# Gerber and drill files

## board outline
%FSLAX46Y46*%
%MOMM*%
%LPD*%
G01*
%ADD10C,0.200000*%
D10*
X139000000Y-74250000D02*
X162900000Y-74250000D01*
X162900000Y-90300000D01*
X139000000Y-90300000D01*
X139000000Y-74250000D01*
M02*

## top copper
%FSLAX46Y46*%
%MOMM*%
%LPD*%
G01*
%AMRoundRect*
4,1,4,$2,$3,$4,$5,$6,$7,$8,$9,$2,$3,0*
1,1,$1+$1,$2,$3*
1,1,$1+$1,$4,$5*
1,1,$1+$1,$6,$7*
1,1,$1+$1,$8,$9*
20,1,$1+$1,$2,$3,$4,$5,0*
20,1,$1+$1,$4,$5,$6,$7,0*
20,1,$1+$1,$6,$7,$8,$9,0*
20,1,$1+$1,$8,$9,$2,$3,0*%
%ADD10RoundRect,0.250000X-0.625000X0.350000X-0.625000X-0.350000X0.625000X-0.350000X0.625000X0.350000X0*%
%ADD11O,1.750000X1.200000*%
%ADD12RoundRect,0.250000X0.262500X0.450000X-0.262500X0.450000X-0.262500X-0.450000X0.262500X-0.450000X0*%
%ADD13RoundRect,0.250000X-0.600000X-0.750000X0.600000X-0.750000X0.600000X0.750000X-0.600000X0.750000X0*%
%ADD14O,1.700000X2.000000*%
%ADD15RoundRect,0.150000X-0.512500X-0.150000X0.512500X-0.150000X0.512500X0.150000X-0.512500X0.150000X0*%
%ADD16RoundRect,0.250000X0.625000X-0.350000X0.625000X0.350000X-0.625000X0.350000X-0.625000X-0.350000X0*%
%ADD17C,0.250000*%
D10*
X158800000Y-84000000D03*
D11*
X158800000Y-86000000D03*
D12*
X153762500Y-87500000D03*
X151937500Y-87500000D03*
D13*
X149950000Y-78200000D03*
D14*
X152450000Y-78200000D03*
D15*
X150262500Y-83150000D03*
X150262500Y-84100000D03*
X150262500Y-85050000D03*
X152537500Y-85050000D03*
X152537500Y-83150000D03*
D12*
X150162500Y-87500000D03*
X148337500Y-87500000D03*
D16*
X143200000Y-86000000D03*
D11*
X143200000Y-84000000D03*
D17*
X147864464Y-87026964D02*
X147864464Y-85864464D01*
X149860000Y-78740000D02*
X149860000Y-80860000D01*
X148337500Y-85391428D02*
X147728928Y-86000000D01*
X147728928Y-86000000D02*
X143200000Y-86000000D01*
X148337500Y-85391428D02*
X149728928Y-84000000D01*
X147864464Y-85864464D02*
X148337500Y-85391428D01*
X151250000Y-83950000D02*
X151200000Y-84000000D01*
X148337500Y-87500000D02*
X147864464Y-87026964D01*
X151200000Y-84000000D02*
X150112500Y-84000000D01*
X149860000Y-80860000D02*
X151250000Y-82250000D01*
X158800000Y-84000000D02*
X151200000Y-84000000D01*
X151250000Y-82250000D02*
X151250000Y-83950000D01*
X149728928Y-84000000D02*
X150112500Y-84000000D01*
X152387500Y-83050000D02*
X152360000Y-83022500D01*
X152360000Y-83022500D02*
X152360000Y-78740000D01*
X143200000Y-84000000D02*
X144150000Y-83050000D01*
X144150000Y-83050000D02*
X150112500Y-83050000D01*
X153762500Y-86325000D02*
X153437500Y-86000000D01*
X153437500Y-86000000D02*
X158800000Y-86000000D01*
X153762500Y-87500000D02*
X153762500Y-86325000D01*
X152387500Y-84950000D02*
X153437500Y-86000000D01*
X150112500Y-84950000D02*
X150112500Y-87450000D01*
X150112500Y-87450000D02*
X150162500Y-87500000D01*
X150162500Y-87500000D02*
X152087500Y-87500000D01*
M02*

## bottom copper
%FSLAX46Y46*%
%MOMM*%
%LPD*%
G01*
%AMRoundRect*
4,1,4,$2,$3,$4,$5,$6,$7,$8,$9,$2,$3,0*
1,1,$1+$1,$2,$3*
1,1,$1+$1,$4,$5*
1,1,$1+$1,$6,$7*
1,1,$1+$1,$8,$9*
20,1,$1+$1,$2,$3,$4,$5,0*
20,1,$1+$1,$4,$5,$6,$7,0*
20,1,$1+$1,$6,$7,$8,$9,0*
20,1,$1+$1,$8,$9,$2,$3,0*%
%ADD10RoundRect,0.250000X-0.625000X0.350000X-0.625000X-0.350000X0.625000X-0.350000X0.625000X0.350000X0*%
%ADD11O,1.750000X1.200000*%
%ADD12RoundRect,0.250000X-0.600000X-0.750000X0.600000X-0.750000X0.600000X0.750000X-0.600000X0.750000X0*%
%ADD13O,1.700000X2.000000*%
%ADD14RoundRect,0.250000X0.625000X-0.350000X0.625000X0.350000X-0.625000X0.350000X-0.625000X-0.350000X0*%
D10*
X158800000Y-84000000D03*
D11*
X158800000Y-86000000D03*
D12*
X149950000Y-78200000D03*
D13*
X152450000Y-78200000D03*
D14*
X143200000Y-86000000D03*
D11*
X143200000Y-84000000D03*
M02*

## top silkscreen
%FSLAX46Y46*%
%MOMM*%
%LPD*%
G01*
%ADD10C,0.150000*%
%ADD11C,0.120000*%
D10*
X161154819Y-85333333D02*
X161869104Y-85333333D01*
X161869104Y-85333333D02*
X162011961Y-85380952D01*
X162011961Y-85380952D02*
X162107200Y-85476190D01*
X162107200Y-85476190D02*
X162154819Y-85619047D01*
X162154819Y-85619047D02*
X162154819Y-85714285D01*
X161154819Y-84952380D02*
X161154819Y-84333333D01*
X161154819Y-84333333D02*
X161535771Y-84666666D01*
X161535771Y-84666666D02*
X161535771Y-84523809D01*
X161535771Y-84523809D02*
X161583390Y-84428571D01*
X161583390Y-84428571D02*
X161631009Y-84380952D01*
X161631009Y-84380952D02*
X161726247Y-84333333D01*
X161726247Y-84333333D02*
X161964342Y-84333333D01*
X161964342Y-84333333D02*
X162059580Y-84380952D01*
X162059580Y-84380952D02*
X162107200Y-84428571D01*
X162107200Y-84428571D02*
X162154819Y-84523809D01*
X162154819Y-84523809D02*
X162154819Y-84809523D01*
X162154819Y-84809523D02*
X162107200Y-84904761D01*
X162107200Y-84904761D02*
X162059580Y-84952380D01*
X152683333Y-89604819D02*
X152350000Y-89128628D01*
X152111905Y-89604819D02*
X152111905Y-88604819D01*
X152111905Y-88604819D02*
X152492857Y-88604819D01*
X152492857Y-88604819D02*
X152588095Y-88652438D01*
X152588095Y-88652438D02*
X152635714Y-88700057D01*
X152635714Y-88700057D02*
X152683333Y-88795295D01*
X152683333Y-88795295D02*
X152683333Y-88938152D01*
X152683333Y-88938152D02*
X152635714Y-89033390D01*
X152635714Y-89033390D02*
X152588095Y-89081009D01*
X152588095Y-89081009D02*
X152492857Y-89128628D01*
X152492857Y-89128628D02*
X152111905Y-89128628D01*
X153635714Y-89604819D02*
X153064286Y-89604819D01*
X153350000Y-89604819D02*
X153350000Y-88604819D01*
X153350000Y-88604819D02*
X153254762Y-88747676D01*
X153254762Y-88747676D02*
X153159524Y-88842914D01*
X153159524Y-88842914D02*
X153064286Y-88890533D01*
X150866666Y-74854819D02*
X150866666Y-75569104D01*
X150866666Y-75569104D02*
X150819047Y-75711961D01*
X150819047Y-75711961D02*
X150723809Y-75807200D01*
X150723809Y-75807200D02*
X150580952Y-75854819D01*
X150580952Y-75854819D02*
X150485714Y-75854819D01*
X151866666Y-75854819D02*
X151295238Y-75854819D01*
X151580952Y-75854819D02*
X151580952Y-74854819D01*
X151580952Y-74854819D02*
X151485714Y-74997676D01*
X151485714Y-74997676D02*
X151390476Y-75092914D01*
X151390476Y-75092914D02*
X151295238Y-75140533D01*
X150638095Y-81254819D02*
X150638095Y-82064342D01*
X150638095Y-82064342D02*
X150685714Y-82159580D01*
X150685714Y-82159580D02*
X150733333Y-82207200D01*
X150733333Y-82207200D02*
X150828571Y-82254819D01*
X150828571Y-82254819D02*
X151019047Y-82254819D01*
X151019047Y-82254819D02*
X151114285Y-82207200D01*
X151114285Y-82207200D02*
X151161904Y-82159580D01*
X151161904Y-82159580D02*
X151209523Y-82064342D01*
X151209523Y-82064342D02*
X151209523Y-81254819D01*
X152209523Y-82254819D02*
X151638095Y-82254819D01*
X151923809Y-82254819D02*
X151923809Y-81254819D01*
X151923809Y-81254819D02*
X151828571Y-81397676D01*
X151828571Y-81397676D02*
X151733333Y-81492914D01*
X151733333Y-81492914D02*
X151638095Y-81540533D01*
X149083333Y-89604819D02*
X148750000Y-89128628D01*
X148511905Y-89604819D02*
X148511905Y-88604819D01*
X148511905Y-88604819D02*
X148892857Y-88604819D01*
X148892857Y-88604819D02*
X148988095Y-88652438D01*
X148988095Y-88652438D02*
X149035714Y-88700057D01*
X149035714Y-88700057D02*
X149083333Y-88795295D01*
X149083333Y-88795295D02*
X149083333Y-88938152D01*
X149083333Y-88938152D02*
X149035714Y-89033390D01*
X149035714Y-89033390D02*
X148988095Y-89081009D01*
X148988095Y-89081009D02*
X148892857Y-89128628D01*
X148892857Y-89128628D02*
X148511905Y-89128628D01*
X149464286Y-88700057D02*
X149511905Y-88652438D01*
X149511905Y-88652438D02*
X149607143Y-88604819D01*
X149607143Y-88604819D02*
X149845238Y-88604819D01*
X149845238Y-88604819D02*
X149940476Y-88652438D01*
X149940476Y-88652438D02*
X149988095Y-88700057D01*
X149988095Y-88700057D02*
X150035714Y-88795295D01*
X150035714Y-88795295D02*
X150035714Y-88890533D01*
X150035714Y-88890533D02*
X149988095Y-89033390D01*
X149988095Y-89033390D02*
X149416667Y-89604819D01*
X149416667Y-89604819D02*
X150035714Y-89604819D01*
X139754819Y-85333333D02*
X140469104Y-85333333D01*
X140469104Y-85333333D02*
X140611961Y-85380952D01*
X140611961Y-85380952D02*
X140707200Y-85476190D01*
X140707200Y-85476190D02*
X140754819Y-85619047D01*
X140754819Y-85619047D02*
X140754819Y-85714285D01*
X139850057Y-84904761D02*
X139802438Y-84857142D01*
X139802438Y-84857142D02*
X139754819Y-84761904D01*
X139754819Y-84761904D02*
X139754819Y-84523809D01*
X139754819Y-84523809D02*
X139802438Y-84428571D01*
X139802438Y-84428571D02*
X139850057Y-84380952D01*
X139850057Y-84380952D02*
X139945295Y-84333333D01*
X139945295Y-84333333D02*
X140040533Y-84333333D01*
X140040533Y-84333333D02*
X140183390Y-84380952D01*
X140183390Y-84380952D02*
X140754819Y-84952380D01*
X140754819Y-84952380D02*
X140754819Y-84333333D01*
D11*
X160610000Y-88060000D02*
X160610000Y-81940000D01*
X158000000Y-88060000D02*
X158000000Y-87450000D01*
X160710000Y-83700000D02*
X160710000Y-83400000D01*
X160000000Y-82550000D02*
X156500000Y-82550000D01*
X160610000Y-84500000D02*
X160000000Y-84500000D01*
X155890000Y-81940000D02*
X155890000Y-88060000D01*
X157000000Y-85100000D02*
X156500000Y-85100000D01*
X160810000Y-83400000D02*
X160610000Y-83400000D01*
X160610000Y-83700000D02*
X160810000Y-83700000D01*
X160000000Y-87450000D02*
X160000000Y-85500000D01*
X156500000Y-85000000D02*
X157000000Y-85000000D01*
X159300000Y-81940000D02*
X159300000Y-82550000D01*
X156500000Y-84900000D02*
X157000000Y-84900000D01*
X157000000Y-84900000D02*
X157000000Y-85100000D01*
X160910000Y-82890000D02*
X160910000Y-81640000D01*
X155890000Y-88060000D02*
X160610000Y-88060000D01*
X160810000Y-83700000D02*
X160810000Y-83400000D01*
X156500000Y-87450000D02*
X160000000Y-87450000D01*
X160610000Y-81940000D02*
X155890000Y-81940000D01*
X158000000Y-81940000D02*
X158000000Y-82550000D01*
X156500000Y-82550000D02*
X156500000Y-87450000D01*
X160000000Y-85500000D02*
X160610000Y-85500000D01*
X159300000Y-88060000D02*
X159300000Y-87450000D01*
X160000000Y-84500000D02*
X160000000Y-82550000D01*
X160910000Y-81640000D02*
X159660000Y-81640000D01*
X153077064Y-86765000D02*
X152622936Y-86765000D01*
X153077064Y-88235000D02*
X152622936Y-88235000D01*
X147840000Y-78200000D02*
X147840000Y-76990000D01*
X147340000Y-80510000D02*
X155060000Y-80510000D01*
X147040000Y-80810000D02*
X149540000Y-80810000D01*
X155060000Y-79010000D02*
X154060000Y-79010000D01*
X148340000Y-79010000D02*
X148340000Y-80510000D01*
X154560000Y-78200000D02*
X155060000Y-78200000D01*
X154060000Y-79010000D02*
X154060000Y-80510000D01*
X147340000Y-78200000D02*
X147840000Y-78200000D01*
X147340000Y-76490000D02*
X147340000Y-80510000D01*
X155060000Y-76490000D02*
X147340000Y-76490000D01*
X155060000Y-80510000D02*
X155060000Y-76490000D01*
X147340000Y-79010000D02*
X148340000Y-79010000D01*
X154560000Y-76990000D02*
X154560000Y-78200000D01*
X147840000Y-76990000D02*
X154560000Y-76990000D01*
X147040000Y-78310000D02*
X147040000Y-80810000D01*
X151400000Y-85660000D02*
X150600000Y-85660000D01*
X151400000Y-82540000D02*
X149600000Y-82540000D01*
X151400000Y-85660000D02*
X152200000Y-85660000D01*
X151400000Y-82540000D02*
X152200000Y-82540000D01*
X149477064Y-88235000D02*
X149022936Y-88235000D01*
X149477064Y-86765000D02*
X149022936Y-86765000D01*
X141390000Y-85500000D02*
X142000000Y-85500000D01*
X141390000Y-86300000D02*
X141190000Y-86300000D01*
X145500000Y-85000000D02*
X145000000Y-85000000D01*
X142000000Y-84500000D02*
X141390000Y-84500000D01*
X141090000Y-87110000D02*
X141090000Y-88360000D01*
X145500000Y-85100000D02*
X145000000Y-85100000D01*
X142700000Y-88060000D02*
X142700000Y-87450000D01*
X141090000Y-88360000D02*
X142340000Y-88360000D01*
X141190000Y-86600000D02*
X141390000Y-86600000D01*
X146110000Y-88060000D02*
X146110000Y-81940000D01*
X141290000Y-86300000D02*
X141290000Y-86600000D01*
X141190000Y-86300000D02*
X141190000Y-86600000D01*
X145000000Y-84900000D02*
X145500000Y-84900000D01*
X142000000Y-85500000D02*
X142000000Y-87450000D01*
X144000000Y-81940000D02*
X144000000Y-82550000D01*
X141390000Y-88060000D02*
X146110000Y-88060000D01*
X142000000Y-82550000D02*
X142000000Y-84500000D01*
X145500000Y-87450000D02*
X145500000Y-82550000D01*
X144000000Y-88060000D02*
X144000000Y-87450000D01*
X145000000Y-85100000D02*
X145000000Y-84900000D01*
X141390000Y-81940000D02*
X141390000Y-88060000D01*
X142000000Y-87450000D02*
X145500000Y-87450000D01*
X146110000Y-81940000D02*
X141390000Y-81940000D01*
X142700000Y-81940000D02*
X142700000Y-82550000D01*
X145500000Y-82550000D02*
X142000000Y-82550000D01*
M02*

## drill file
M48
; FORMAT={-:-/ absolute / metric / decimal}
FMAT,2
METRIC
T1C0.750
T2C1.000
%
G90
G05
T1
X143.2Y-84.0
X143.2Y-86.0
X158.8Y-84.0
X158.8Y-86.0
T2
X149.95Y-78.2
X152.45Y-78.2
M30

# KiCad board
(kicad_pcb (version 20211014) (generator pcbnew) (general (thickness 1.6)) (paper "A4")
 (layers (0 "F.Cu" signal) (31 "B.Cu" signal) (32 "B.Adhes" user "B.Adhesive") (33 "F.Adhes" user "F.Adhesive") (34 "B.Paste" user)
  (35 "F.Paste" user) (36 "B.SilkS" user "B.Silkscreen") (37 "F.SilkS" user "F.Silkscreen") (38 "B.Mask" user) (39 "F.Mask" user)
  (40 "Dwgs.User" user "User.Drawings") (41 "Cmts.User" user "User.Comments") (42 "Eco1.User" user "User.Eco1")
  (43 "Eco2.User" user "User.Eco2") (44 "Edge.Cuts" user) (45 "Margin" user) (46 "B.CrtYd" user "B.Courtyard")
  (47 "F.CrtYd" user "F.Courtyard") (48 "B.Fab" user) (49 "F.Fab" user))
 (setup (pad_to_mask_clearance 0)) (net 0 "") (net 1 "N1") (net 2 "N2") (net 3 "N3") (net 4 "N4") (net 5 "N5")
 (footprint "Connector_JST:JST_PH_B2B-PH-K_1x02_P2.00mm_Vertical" (layer "F.Cu") (at 158.8 84 -90)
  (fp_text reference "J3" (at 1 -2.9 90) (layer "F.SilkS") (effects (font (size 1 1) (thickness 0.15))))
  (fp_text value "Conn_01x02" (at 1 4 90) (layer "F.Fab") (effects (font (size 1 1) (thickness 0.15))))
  (fp_line (start 4.06 -1.81) (end -2.06 -1.81) (layer "F.SilkS") (width 0.12))
  (fp_line (start 4.06 0.8) (end 3.45 0.8) (layer "F.SilkS") (width 0.12))
  (fp_line (start -0.3 -1.91) (end -0.6 -1.91) (layer "F.SilkS") (width 0.12))
  (fp_line (start -1.45 -1.2) (end -1.45 2.3) (layer "F.SilkS") (width 0.12))
  (fp_line (start 0.5 -1.81) (end 0.5 -1.2) (layer "F.SilkS") (width 0.12))
  (fp_line (start -2.06 2.91) (end 4.06 2.91) (layer "F.SilkS") (width 0.12))
  (fp_line (start 1.1 1.8) (end 1.1 2.3) (layer "F.SilkS") (width 0.12))
  (fp_line (start -0.6 -2.01) (end -0.6 -1.81) (layer "F.SilkS") (width 0.12))
  (fp_line (start -0.3 -1.81) (end -0.3 -2.01) (layer "F.SilkS") (width 0.12))
  (fp_line (start 3.45 -1.2) (end 1.5 -1.2) (layer "F.SilkS") (width 0.12))
  (fp_line (start 1 2.3) (end 1 1.8) (layer "F.SilkS") (width 0.12))
  (fp_line (start -2.06 -0.5) (end -1.45 -0.5) (layer "F.SilkS") (width 0.12))
  (fp_line (start 0.9 2.3) (end 0.9 1.8) (layer "F.SilkS") (width 0.12))
  (fp_line (start 0.9 1.8) (end 1.1 1.8) (layer "F.SilkS") (width 0.12))
  (fp_line (start -1.11 -2.11) (end -2.36 -2.11) (layer "F.SilkS") (width 0.12))
  (fp_line (start 4.06 2.91) (end 4.06 -1.81) (layer "F.SilkS") (width 0.12))
  (fp_line (start -0.3 -2.01) (end -0.6 -2.01) (layer "F.SilkS") (width 0.12))
  (fp_line (start 3.45 2.3) (end 3.45 -1.2) (layer "F.SilkS") (width 0.12))
  (fp_line (start -2.06 -1.81) (end -2.06 2.91) (layer "F.SilkS") (width 0.12))
  (fp_line (start -2.06 0.8) (end -1.45 0.8) (layer "F.SilkS") (width 0.12))
  (fp_line (start -1.45 2.3) (end 3.45 2.3) (layer "F.SilkS") (width 0.12))
  (fp_line (start 1.5 -1.2) (end 1.5 -1.81) (layer "F.SilkS") (width 0.12))
  (fp_line (start 4.06 -0.5) (end 3.45 -0.5) (layer "F.SilkS") (width 0.12))
  (fp_line (start 0.5 -1.2) (end -1.45 -1.2) (layer "F.SilkS") (width 0.12))
  (fp_line (start -2.36 -2.11) (end -2.36 -0.86) (layer "F.SilkS") (width 0.12))
  (pad "1" thru_hole roundrect locked (at 0 0 270) (size 1.2 1.75) (drill 0.75) (layers *.Cu *.Mask) (roundrect_rratio 0.208333)
   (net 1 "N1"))
  (pad "2" thru_hole oval locked (at 2 0 270) (size 1.2 1.75) (drill 0.75) (layers *.Cu *.Mask) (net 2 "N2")))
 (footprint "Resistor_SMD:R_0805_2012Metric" (layer "F.Cu") (at 152.85 87.5 180)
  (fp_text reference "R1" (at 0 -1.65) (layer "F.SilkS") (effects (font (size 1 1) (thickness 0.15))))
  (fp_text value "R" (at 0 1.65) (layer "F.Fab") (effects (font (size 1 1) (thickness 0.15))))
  (fp_line (start -0.227064 0.735) (end 0.227064 0.735) (layer "F.SilkS") (width 0.12))
  (fp_line (start -0.227064 -0.735) (end 0.227064 -0.735) (layer "F.SilkS") (width 0.12))
  (pad "1" smd roundrect locked (at -0.9125 0 180) (size 1.025 1.4) (layers "F.Cu" "F.Paste" "F.Mask") (roundrect_rratio 0.243902)
   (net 2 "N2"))
  (pad "2" smd roundrect locked (at 0.9125 0 180) (size 1.025 1.4) (layers "F.Cu" "F.Paste" "F.Mask") (roundrect_rratio 0.243902)
   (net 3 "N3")))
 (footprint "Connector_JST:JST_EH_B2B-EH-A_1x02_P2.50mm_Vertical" (layer "F.Cu") (at 149.95 78.2)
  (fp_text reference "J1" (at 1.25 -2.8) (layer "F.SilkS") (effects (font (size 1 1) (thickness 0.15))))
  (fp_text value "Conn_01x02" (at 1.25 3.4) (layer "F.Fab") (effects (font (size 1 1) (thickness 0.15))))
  (fp_line (start -2.11 0) (end -2.11 -1.21) (layer "F.SilkS") (width 0.12))
  (fp_line (start -2.61 2.31) (end 5.11 2.31) (layer "F.SilkS") (width 0.12))
  (fp_line (start -2.91 2.61) (end -0.41 2.61) (layer "F.SilkS") (width 0.12))
  (fp_line (start 5.11 0.81) (end 4.11 0.81) (layer "F.SilkS") (width 0.12))
  (fp_line (start -1.61 0.81) (end -1.61 2.31) (layer "F.SilkS") (width 0.12))
  (fp_line (start 4.61 0) (end 5.11 0) (layer "F.SilkS") (width 0.12))
  (fp_line (start 4.11 0.81) (end 4.11 2.31) (layer "F.SilkS") (width 0.12))
  (fp_line (start -2.61 0) (end -2.11 0) (layer "F.SilkS") (width 0.12))
  (fp_line (start -2.61 -1.71) (end -2.61 2.31) (layer "F.SilkS") (width 0.12))
  (fp_line (start 5.11 -1.71) (end -2.61 -1.71) (layer "F.SilkS") (width 0.12))
  (fp_line (start 5.11 2.31) (end 5.11 -1.71) (layer "F.SilkS") (width 0.12))
  (fp_line (start -2.61 0.81) (end -1.61 0.81) (layer "F.SilkS") (width 0.12))
  (fp_line (start 4.61 -1.21) (end 4.61 0) (layer "F.SilkS") (width 0.12))
  (fp_line (start -2.11 -1.21) (end 4.61 -1.21) (layer "F.SilkS") (width 0.12))
  (fp_line (start -2.91 0.11) (end -2.91 2.61) (layer "F.SilkS") (width 0.12))
  (pad "1" thru_hole roundrect locked (at 0 0) (size 1.7 2) (drill 1) (layers *.Cu *.Mask) (roundrect_rratio 0.147059) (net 1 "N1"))
  (pad "2" thru_hole oval locked (at 2.5 0) (size 1.7 2) (drill 1) (layers *.Cu *.Mask) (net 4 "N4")))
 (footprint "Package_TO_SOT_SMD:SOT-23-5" (layer "F.Cu") (at 151.4 84.1)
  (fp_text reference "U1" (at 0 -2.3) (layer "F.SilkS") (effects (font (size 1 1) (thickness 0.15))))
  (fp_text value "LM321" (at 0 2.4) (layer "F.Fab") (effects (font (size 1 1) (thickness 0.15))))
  (fp_line (start 0 1.56) (end -0.8 1.56) (layer "F.SilkS") (width 0.12))
  (fp_line (start 0 -1.56) (end -1.8 -1.56) (layer "F.SilkS") (width 0.12))
  (fp_line (start 0 1.56) (end 0.8 1.56) (layer "F.SilkS") (width 0.12))
  (fp_line (start 0 -1.56) (end 0.8 -1.56) (layer "F.SilkS") (width 0.12))
  (pad "1" smd roundrect locked (at -1.1375 -0.95) (size 1.325 0.6) (layers "F.Cu" "F.Paste" "F.Mask") (roundrect_rratio 0.25) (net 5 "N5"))
  (pad "2" smd roundrect locked (at -1.1375 0) (size 1.325 0.6) (layers "F.Cu" "F.Paste" "F.Mask") (roundrect_rratio 0.25) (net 1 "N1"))
  (pad "3" smd roundrect locked (at -1.1375 0.95) (size 1.325 0.6) (layers "F.Cu" "F.Paste" "F.Mask") (roundrect_rratio 0.25) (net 3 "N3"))
  (pad "4" smd roundrect locked (at 1.1375 0.95) (size 1.325 0.6) (layers "F.Cu" "F.Paste" "F.Mask") (roundrect_rratio 0.25) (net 2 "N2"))
  (pad "5" smd roundrect locked (at 1.1375 -0.95) (size 1.325 0.6) (layers "F.Cu" "F.Paste" "F.Mask") (roundrect_rratio 0.25) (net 4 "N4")))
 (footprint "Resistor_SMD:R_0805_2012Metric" (layer "F.Cu") (at 149.25 87.5 180)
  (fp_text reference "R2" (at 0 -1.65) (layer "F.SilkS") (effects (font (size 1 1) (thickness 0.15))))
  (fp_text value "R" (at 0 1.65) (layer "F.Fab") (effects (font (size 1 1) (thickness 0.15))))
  (fp_line (start -0.227064 -0.735) (end 0.227064 -0.735) (layer "F.SilkS") (width 0.12))
  (fp_line (start -0.227064 0.735) (end 0.227064 0.735) (layer "F.SilkS") (width 0.12))
  (pad "1" smd roundrect locked (at -0.9125 0 180) (size 1.025 1.4) (layers "F.Cu" "F.Paste" "F.Mask") (roundrect_rratio 0.243902)
   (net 3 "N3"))
  (pad "2" smd roundrect locked (at 0.9125 0 180) (size 1.025 1.4) (layers "F.Cu" "F.Paste" "F.Mask") (roundrect_rratio 0.243902)
   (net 1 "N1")))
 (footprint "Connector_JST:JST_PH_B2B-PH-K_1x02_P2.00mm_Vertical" (layer "F.Cu") (at 143.2 86 90)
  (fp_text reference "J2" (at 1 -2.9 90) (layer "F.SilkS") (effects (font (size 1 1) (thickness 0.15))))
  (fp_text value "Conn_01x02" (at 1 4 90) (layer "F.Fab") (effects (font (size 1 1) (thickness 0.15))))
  (fp_line (start 0.5 -1.81) (end 0.5 -1.2) (layer "F.SilkS") (width 0.12))
  (fp_line (start -0.3 -1.81) (end -0.3 -2.01) (layer "F.SilkS") (width 0.12))
  (fp_line (start 1 2.3) (end 1 1.8) (layer "F.SilkS") (width 0.12))
  (fp_line (start 1.5 -1.2) (end 1.5 -1.81) (layer "F.SilkS") (width 0.12))
  (fp_line (start -1.11 -2.11) (end -2.36 -2.11) (layer "F.SilkS") (width 0.12))
  (fp_line (start 0.9 2.3) (end 0.9 1.8) (layer "F.SilkS") (width 0.12))
  (fp_line (start -2.06 -0.5) (end -1.45 -0.5) (layer "F.SilkS") (width 0.12))
  (fp_line (start -2.36 -2.11) (end -2.36 -0.86) (layer "F.SilkS") (width 0.12))
  (fp_line (start -0.6 -2.01) (end -0.6 -1.81) (layer "F.SilkS") (width 0.12))
  (fp_line (start -2.06 2.91) (end 4.06 2.91) (layer "F.SilkS") (width 0.12))
  (fp_line (start -0.3 -1.91) (end -0.6 -1.91) (layer "F.SilkS") (width 0.12))
  (fp_line (start -0.3 -2.01) (end -0.6 -2.01) (layer "F.SilkS") (width 0.12))
  (fp_line (start 1.1 1.8) (end 1.1 2.3) (layer "F.SilkS") (width 0.12))
  (fp_line (start 0.5 -1.2) (end -1.45 -1.2) (layer "F.SilkS") (width 0.12))
  (fp_line (start 4.06 0.8) (end 3.45 0.8) (layer "F.SilkS") (width 0.12))
  (fp_line (start -2.06 -1.81) (end -2.06 2.91) (layer "F.SilkS") (width 0.12))
  (fp_line (start 3.45 -1.2) (end 1.5 -1.2) (layer "F.SilkS") (width 0.12))
  (fp_line (start -1.45 2.3) (end 3.45 2.3) (layer "F.SilkS") (width 0.12))
  (fp_line (start -2.06 0.8) (end -1.45 0.8) (layer "F.SilkS") (width 0.12))
  (fp_line (start 0.9 1.8) (end 1.1 1.8) (layer "F.SilkS") (width 0.12))
  (fp_line (start 4.06 -1.81) (end -2.06 -1.81) (layer "F.SilkS") (width 0.12))
  (fp_line (start -1.45 -1.2) (end -1.45 2.3) (layer "F.SilkS") (width 0.12))
  (fp_line (start 4.06 2.91) (end 4.06 -1.81) (layer "F.SilkS") (width 0.12))
  (fp_line (start 4.06 -0.5) (end 3.45 -0.5) (layer "F.SilkS") (width 0.12))
  (fp_line (start 3.45 2.3) (end 3.45 -1.2) (layer "F.SilkS") (width 0.12))
  (pad "1" thru_hole roundrect locked (at 0 0 90) (size 1.2 1.75) (drill 0.75) (layers *.Cu *.Mask) (roundrect_rratio 0.208333) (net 1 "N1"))
  (pad "2" thru_hole oval locked (at 2 0 90) (size 1.2 1.75) (drill 0.75) (layers *.Cu *.Mask) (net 5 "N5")))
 (gr_rect (start 162.9 90.3) (end 139 74.25) (layer "Edge.Cuts") (width 0.2) (fill none))
 (segment (start 147.864464 87.026964) (end 147.864464 85.864464) (width 0.25) (layer "F.Cu") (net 1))
 (segment (start 149.86 78.74) (end 149.86 80.86) (width 0.25) (layer "F.Cu") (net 1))
 (segment (start 148.3375 85.391428) (end 147.728928 86) (width 0.25) (layer "F.Cu") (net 1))
 (segment (start 147.728928 86) (end 143.2 86) (width 0.25) (layer "F.Cu") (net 1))
 (segment (start 148.3375 85.391428) (end 149.728928 84) (width 0.25) (layer "F.Cu") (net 1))
 (segment (start 147.864464 85.864464) (end 148.3375 85.391428) (width 0.25) (layer "F.Cu") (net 1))
 (segment (start 151.25 83.95) (end 151.2 84) (width 0.25) (layer "F.Cu") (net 1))
 (segment (start 148.3375 87.5) (end 147.864464 87.026964) (width 0.25) (layer "F.Cu") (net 1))
 (segment (start 151.2 84) (end 150.1125 84) (width 0.25) (layer "F.Cu") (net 1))
 (segment (start 149.86 80.86) (end 151.25 82.25) (width 0.25) (layer "F.Cu") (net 1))
 (segment (start 158.8 84) (end 151.2 84) (width 0.25) (layer "F.Cu") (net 1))
 (segment (start 151.25 82.25) (end 151.25 83.95) (width 0.25) (layer "F.Cu") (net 1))
 (segment (start 149.728928 84) (end 150.1125 84) (width 0.25) (layer "F.Cu") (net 1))
 (segment (start 152.3875 83.05) (end 152.36 83.0225) (width 0.25) (layer "F.Cu") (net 4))
 (segment (start 152.36 83.0225) (end 152.36 78.74) (width 0.25) (layer "F.Cu") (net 4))
 (segment (start 143.2 84) (end 144.15 83.05) (width 0.25) (layer "F.Cu") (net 5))
 (segment (start 144.15 83.05) (end 150.1125 83.05) (width 0.25) (layer "F.Cu") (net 5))
 (segment (start 153.7625 86.325) (end 153.4375 86) (width 0.25) (layer "F.Cu") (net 2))
 (segment (start 153.4375 86) (end 158.8 86) (width 0.25) (layer "F.Cu") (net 2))
 (segment (start 153.7625 87.5) (end 153.7625 86.325) (width 0.25) (layer "F.Cu") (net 2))
 (segment (start 152.3875 84.95) (end 153.4375 86) (width 0.25) (layer "F.Cu") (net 2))
 (segment (start 150.1125 84.95) (end 150.1125 87.45) (width 0.25) (layer "F.Cu") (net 3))
 (segment (start 150.1125 87.45) (end 150.1625 87.5) (width 0.25) (layer "F.Cu") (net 3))
 (segment (start 150.1625 87.5) (end 152.0875 87.5) (width 0.25) (layer "F.Cu") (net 3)))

